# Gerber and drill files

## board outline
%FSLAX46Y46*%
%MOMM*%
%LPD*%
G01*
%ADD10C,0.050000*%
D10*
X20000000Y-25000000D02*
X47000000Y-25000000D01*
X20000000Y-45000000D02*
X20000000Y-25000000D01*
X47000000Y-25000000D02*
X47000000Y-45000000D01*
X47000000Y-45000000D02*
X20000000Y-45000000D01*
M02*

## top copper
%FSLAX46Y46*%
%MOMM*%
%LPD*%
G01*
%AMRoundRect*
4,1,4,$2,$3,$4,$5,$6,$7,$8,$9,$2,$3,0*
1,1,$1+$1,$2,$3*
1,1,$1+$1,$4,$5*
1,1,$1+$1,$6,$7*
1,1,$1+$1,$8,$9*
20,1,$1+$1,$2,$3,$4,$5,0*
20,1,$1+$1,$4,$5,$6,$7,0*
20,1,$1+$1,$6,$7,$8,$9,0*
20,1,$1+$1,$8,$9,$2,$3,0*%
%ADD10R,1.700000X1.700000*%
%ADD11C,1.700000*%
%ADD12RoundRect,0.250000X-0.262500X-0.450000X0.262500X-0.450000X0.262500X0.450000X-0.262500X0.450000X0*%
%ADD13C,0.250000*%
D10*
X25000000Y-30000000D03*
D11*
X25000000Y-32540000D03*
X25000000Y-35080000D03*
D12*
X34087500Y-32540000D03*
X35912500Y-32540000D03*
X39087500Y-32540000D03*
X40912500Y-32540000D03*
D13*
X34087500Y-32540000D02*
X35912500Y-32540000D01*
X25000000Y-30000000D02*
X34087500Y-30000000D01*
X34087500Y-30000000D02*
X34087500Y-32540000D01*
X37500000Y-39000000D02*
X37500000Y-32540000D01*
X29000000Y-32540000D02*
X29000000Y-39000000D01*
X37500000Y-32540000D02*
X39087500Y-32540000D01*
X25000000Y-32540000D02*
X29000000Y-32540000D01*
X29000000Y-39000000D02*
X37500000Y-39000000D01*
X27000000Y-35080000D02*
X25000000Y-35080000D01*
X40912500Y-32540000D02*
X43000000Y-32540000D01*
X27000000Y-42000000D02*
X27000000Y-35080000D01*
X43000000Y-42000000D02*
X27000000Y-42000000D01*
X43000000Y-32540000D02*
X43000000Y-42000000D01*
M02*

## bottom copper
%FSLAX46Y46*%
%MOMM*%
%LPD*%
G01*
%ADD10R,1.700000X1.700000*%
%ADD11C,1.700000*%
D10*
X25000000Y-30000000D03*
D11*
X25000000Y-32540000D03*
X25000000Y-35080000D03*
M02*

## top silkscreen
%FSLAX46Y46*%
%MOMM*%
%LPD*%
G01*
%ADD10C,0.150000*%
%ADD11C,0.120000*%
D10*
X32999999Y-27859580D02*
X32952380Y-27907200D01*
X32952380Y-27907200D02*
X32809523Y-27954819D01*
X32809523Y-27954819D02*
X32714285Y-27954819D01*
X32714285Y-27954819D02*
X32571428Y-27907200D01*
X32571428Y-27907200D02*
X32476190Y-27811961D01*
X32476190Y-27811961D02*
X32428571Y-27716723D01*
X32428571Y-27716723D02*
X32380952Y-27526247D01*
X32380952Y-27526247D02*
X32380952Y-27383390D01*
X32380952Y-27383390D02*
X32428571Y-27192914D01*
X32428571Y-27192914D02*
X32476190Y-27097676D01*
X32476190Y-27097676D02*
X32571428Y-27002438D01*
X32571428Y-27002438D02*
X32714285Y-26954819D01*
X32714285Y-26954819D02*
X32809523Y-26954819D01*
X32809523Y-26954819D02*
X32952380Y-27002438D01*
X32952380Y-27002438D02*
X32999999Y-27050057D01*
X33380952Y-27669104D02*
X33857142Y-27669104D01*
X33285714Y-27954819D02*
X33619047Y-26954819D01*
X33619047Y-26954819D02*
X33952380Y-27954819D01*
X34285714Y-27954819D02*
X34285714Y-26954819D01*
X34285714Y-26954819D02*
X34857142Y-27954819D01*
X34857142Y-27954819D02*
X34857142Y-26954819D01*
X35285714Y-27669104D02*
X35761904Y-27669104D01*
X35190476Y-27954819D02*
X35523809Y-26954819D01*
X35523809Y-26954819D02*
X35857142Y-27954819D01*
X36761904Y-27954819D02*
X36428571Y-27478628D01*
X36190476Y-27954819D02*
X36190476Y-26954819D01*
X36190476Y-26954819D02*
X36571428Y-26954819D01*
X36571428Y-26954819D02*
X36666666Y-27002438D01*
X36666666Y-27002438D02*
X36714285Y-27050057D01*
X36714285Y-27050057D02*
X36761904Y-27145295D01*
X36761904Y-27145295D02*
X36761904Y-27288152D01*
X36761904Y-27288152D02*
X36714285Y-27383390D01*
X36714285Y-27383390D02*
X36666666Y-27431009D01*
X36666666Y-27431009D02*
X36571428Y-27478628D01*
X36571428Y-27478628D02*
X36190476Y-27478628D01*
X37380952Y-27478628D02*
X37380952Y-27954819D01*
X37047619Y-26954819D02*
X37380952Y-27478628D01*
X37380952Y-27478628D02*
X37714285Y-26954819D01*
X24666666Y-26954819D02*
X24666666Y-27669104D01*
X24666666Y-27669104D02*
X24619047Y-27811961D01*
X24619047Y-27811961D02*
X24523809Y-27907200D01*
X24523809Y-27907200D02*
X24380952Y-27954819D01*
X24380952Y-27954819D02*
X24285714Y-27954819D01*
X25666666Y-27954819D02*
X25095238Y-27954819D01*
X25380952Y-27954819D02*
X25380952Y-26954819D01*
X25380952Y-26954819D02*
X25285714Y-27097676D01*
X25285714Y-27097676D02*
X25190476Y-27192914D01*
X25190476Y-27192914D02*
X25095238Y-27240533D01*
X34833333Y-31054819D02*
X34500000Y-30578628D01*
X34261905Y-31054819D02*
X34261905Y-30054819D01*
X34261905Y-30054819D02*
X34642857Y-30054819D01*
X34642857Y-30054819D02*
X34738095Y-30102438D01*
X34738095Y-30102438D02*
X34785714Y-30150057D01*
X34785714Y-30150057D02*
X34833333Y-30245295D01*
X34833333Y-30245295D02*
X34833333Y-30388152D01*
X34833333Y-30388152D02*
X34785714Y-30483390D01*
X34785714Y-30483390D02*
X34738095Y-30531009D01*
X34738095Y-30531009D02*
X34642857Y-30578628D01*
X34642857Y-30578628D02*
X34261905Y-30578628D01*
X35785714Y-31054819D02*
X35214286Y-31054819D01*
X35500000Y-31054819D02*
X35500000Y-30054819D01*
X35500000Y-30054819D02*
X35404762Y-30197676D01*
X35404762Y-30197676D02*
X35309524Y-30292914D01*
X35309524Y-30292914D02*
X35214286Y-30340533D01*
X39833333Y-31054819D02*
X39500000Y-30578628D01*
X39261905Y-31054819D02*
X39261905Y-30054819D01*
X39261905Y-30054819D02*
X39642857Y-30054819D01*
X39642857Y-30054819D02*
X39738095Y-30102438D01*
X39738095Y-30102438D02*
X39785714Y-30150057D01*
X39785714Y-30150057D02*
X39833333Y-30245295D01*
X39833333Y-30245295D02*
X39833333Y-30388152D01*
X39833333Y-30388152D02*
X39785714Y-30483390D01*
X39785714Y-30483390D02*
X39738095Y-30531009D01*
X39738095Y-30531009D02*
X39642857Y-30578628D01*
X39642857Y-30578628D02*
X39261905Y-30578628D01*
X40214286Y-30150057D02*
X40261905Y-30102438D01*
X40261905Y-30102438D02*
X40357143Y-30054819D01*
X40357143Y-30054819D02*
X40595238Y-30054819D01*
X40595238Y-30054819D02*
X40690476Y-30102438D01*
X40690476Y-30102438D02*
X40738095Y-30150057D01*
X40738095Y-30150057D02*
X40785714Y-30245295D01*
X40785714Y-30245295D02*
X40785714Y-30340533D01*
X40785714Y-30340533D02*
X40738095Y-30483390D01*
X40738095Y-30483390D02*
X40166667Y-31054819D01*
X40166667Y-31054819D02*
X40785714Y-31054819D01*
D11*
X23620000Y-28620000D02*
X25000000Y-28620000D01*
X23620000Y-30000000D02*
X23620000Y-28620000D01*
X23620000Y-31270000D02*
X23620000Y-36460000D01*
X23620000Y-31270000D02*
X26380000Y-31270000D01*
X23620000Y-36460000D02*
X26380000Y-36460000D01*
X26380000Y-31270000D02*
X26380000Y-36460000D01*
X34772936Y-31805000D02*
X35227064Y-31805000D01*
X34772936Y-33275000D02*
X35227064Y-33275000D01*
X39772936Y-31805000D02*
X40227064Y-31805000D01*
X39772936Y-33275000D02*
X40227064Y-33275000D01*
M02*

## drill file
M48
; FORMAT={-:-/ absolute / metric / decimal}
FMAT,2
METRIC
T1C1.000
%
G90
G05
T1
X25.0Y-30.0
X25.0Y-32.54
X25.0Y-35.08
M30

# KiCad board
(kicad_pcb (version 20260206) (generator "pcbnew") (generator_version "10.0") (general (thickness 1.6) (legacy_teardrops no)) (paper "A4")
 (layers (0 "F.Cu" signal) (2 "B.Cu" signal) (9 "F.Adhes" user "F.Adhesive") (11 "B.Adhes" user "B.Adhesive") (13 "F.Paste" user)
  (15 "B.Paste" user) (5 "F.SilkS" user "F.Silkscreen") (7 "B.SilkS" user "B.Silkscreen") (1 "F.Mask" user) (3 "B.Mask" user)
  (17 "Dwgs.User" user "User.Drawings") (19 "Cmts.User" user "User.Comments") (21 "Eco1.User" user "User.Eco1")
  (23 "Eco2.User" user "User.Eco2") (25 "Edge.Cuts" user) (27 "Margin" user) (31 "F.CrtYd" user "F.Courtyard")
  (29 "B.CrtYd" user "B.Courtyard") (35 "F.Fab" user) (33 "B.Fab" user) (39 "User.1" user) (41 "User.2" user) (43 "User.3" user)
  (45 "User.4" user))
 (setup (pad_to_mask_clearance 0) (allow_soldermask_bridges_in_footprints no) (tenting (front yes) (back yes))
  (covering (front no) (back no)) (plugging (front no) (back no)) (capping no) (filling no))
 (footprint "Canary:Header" (layer "F.Cu") (at 25 30)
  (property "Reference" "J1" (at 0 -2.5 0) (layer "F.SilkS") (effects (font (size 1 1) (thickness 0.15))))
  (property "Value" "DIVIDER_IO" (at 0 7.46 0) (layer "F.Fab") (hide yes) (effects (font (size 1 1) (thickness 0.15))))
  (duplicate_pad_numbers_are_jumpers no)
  (fp_line (start -1.38 -1.38) (end 0 -1.38) (stroke (width 0.12) (type solid)) (layer "F.SilkS"))
  (fp_line (start -1.38 0) (end -1.38 -1.38) (stroke (width 0.12) (type solid)) (layer "F.SilkS"))
  (fp_line (start -1.38 1.27) (end -1.38 6.46) (stroke (width 0.12) (type solid)) (layer "F.SilkS"))
  (fp_line (start -1.38 1.27) (end 1.38 1.27) (stroke (width 0.12) (type solid)) (layer "F.SilkS"))
  (fp_line (start -1.38 6.46) (end 1.38 6.46) (stroke (width 0.12) (type solid)) (layer "F.SilkS"))
  (fp_line (start 1.38 1.27) (end 1.38 6.46) (stroke (width 0.12) (type solid)) (layer "F.SilkS"))
  (pad "1" thru_hole rect (at 0 0) (size 1.7 1.7) (drill 1) (layers "*.Cu" "*.Mask") (remove_unused_layers no) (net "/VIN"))
  (pad "2" thru_hole circle (at 0 2.54) (size 1.7 1.7) (drill 1) (layers "*.Cu" "*.Mask") (remove_unused_layers no) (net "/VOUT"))
  (pad "3" thru_hole circle (at 0 5.08) (size 1.7 1.7) (drill 1) (layers "*.Cu" "*.Mask") (remove_unused_layers no) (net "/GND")))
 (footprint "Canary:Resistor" (layer "F.Cu") (at 35 32.54)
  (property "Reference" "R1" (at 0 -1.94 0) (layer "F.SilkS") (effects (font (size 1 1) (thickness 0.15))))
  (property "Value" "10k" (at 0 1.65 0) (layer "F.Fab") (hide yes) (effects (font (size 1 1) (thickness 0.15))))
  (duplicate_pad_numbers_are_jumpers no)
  (fp_line (start -0.227064 -0.735) (end 0.227064 -0.735) (stroke (width 0.12) (type solid)) (layer "F.SilkS"))
  (fp_line (start -0.227064 0.735) (end 0.227064 0.735) (stroke (width 0.12) (type solid)) (layer "F.SilkS"))
  (pad "1" smd roundrect (at -0.9125 0) (size 1.025 1.4) (layers "F.Cu" "F.Mask" "F.Paste") (roundrect_rratio 0.243902) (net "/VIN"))
  (pad "2" smd roundrect (at 0.9125 0) (size 1.025 1.4) (layers "F.Cu" "F.Mask" "F.Paste") (roundrect_rratio 0.243902) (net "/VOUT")))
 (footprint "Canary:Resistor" (layer "F.Cu") (at 40 32.54)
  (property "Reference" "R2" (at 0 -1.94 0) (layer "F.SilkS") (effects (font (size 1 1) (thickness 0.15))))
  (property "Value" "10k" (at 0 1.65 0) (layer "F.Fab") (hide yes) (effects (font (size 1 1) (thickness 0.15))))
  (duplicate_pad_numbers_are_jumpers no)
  (fp_line (start -0.227064 -0.735) (end 0.227064 -0.735) (stroke (width 0.12) (type solid)) (layer "F.SilkS"))
  (fp_line (start -0.227064 0.735) (end 0.227064 0.735) (stroke (width 0.12) (type solid)) (layer "F.SilkS"))
  (pad "1" smd roundrect (at -0.9125 0) (size 1.025 1.4) (layers "F.Cu" "F.Mask" "F.Paste") (roundrect_rratio 0.243902) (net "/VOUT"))
  (pad "2" smd roundrect (at 0.9125 0) (size 1.025 1.4) (layers "F.Cu" "F.Mask" "F.Paste") (roundrect_rratio 0.243902) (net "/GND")))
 (gr_line (start 20 25) (end 47 25) (stroke (width 0.05) (type default)) (layer "Edge.Cuts"))
 (gr_line (start 20 45) (end 20 25) (stroke (width 0.05) (type default)) (layer "Edge.Cuts"))
 (gr_line (start 47 25) (end 47 45) (stroke (width 0.05) (type default)) (layer "Edge.Cuts"))
 (gr_line (start 47 45) (end 20 45) (stroke (width 0.05) (type default)) (layer "Edge.Cuts"))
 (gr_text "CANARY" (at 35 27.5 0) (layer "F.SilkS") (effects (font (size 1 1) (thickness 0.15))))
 (segment (start 34.0875 32.54) (end 35.9125 32.54) (width 0.25) (layer "F.Cu") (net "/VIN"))
 (segment (start 25 30) (end 34.0875 30) (width 0.25) (layer "F.Cu") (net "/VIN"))
 (segment (start 34.0875 30) (end 34.0875 32.54) (width 0.25) (layer "F.Cu") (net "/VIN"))
 (segment (start 37.5 39) (end 37.5 32.54) (width 0.25) (layer "F.Cu") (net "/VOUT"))
 (segment (start 29 32.54) (end 29 39) (width 0.25) (layer "F.Cu") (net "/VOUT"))
 (segment (start 37.5 32.54) (end 39.0875 32.54) (width 0.25) (layer "F.Cu") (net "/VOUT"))
 (segment (start 25 32.54) (end 29 32.54) (width 0.25) (layer "F.Cu") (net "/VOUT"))
 (segment (start 29 39) (end 37.5 39) (width 0.25) (layer "F.Cu") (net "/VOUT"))
 (segment (start 27 35.08) (end 25 35.08) (width 0.25) (layer "F.Cu") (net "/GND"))
 (segment (start 40.9125 32.54) (end 43 32.54) (width 0.25) (layer "F.Cu") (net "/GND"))
 (segment (start 27 42) (end 27 35.08) (width 0.25) (layer "F.Cu") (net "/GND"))
 (segment (start 43 42) (end 27 42) (width 0.25) (layer "F.Cu") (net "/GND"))
 (segment (start 43 32.54) (end 43 42) (width 0.25) (layer "F.Cu") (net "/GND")))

